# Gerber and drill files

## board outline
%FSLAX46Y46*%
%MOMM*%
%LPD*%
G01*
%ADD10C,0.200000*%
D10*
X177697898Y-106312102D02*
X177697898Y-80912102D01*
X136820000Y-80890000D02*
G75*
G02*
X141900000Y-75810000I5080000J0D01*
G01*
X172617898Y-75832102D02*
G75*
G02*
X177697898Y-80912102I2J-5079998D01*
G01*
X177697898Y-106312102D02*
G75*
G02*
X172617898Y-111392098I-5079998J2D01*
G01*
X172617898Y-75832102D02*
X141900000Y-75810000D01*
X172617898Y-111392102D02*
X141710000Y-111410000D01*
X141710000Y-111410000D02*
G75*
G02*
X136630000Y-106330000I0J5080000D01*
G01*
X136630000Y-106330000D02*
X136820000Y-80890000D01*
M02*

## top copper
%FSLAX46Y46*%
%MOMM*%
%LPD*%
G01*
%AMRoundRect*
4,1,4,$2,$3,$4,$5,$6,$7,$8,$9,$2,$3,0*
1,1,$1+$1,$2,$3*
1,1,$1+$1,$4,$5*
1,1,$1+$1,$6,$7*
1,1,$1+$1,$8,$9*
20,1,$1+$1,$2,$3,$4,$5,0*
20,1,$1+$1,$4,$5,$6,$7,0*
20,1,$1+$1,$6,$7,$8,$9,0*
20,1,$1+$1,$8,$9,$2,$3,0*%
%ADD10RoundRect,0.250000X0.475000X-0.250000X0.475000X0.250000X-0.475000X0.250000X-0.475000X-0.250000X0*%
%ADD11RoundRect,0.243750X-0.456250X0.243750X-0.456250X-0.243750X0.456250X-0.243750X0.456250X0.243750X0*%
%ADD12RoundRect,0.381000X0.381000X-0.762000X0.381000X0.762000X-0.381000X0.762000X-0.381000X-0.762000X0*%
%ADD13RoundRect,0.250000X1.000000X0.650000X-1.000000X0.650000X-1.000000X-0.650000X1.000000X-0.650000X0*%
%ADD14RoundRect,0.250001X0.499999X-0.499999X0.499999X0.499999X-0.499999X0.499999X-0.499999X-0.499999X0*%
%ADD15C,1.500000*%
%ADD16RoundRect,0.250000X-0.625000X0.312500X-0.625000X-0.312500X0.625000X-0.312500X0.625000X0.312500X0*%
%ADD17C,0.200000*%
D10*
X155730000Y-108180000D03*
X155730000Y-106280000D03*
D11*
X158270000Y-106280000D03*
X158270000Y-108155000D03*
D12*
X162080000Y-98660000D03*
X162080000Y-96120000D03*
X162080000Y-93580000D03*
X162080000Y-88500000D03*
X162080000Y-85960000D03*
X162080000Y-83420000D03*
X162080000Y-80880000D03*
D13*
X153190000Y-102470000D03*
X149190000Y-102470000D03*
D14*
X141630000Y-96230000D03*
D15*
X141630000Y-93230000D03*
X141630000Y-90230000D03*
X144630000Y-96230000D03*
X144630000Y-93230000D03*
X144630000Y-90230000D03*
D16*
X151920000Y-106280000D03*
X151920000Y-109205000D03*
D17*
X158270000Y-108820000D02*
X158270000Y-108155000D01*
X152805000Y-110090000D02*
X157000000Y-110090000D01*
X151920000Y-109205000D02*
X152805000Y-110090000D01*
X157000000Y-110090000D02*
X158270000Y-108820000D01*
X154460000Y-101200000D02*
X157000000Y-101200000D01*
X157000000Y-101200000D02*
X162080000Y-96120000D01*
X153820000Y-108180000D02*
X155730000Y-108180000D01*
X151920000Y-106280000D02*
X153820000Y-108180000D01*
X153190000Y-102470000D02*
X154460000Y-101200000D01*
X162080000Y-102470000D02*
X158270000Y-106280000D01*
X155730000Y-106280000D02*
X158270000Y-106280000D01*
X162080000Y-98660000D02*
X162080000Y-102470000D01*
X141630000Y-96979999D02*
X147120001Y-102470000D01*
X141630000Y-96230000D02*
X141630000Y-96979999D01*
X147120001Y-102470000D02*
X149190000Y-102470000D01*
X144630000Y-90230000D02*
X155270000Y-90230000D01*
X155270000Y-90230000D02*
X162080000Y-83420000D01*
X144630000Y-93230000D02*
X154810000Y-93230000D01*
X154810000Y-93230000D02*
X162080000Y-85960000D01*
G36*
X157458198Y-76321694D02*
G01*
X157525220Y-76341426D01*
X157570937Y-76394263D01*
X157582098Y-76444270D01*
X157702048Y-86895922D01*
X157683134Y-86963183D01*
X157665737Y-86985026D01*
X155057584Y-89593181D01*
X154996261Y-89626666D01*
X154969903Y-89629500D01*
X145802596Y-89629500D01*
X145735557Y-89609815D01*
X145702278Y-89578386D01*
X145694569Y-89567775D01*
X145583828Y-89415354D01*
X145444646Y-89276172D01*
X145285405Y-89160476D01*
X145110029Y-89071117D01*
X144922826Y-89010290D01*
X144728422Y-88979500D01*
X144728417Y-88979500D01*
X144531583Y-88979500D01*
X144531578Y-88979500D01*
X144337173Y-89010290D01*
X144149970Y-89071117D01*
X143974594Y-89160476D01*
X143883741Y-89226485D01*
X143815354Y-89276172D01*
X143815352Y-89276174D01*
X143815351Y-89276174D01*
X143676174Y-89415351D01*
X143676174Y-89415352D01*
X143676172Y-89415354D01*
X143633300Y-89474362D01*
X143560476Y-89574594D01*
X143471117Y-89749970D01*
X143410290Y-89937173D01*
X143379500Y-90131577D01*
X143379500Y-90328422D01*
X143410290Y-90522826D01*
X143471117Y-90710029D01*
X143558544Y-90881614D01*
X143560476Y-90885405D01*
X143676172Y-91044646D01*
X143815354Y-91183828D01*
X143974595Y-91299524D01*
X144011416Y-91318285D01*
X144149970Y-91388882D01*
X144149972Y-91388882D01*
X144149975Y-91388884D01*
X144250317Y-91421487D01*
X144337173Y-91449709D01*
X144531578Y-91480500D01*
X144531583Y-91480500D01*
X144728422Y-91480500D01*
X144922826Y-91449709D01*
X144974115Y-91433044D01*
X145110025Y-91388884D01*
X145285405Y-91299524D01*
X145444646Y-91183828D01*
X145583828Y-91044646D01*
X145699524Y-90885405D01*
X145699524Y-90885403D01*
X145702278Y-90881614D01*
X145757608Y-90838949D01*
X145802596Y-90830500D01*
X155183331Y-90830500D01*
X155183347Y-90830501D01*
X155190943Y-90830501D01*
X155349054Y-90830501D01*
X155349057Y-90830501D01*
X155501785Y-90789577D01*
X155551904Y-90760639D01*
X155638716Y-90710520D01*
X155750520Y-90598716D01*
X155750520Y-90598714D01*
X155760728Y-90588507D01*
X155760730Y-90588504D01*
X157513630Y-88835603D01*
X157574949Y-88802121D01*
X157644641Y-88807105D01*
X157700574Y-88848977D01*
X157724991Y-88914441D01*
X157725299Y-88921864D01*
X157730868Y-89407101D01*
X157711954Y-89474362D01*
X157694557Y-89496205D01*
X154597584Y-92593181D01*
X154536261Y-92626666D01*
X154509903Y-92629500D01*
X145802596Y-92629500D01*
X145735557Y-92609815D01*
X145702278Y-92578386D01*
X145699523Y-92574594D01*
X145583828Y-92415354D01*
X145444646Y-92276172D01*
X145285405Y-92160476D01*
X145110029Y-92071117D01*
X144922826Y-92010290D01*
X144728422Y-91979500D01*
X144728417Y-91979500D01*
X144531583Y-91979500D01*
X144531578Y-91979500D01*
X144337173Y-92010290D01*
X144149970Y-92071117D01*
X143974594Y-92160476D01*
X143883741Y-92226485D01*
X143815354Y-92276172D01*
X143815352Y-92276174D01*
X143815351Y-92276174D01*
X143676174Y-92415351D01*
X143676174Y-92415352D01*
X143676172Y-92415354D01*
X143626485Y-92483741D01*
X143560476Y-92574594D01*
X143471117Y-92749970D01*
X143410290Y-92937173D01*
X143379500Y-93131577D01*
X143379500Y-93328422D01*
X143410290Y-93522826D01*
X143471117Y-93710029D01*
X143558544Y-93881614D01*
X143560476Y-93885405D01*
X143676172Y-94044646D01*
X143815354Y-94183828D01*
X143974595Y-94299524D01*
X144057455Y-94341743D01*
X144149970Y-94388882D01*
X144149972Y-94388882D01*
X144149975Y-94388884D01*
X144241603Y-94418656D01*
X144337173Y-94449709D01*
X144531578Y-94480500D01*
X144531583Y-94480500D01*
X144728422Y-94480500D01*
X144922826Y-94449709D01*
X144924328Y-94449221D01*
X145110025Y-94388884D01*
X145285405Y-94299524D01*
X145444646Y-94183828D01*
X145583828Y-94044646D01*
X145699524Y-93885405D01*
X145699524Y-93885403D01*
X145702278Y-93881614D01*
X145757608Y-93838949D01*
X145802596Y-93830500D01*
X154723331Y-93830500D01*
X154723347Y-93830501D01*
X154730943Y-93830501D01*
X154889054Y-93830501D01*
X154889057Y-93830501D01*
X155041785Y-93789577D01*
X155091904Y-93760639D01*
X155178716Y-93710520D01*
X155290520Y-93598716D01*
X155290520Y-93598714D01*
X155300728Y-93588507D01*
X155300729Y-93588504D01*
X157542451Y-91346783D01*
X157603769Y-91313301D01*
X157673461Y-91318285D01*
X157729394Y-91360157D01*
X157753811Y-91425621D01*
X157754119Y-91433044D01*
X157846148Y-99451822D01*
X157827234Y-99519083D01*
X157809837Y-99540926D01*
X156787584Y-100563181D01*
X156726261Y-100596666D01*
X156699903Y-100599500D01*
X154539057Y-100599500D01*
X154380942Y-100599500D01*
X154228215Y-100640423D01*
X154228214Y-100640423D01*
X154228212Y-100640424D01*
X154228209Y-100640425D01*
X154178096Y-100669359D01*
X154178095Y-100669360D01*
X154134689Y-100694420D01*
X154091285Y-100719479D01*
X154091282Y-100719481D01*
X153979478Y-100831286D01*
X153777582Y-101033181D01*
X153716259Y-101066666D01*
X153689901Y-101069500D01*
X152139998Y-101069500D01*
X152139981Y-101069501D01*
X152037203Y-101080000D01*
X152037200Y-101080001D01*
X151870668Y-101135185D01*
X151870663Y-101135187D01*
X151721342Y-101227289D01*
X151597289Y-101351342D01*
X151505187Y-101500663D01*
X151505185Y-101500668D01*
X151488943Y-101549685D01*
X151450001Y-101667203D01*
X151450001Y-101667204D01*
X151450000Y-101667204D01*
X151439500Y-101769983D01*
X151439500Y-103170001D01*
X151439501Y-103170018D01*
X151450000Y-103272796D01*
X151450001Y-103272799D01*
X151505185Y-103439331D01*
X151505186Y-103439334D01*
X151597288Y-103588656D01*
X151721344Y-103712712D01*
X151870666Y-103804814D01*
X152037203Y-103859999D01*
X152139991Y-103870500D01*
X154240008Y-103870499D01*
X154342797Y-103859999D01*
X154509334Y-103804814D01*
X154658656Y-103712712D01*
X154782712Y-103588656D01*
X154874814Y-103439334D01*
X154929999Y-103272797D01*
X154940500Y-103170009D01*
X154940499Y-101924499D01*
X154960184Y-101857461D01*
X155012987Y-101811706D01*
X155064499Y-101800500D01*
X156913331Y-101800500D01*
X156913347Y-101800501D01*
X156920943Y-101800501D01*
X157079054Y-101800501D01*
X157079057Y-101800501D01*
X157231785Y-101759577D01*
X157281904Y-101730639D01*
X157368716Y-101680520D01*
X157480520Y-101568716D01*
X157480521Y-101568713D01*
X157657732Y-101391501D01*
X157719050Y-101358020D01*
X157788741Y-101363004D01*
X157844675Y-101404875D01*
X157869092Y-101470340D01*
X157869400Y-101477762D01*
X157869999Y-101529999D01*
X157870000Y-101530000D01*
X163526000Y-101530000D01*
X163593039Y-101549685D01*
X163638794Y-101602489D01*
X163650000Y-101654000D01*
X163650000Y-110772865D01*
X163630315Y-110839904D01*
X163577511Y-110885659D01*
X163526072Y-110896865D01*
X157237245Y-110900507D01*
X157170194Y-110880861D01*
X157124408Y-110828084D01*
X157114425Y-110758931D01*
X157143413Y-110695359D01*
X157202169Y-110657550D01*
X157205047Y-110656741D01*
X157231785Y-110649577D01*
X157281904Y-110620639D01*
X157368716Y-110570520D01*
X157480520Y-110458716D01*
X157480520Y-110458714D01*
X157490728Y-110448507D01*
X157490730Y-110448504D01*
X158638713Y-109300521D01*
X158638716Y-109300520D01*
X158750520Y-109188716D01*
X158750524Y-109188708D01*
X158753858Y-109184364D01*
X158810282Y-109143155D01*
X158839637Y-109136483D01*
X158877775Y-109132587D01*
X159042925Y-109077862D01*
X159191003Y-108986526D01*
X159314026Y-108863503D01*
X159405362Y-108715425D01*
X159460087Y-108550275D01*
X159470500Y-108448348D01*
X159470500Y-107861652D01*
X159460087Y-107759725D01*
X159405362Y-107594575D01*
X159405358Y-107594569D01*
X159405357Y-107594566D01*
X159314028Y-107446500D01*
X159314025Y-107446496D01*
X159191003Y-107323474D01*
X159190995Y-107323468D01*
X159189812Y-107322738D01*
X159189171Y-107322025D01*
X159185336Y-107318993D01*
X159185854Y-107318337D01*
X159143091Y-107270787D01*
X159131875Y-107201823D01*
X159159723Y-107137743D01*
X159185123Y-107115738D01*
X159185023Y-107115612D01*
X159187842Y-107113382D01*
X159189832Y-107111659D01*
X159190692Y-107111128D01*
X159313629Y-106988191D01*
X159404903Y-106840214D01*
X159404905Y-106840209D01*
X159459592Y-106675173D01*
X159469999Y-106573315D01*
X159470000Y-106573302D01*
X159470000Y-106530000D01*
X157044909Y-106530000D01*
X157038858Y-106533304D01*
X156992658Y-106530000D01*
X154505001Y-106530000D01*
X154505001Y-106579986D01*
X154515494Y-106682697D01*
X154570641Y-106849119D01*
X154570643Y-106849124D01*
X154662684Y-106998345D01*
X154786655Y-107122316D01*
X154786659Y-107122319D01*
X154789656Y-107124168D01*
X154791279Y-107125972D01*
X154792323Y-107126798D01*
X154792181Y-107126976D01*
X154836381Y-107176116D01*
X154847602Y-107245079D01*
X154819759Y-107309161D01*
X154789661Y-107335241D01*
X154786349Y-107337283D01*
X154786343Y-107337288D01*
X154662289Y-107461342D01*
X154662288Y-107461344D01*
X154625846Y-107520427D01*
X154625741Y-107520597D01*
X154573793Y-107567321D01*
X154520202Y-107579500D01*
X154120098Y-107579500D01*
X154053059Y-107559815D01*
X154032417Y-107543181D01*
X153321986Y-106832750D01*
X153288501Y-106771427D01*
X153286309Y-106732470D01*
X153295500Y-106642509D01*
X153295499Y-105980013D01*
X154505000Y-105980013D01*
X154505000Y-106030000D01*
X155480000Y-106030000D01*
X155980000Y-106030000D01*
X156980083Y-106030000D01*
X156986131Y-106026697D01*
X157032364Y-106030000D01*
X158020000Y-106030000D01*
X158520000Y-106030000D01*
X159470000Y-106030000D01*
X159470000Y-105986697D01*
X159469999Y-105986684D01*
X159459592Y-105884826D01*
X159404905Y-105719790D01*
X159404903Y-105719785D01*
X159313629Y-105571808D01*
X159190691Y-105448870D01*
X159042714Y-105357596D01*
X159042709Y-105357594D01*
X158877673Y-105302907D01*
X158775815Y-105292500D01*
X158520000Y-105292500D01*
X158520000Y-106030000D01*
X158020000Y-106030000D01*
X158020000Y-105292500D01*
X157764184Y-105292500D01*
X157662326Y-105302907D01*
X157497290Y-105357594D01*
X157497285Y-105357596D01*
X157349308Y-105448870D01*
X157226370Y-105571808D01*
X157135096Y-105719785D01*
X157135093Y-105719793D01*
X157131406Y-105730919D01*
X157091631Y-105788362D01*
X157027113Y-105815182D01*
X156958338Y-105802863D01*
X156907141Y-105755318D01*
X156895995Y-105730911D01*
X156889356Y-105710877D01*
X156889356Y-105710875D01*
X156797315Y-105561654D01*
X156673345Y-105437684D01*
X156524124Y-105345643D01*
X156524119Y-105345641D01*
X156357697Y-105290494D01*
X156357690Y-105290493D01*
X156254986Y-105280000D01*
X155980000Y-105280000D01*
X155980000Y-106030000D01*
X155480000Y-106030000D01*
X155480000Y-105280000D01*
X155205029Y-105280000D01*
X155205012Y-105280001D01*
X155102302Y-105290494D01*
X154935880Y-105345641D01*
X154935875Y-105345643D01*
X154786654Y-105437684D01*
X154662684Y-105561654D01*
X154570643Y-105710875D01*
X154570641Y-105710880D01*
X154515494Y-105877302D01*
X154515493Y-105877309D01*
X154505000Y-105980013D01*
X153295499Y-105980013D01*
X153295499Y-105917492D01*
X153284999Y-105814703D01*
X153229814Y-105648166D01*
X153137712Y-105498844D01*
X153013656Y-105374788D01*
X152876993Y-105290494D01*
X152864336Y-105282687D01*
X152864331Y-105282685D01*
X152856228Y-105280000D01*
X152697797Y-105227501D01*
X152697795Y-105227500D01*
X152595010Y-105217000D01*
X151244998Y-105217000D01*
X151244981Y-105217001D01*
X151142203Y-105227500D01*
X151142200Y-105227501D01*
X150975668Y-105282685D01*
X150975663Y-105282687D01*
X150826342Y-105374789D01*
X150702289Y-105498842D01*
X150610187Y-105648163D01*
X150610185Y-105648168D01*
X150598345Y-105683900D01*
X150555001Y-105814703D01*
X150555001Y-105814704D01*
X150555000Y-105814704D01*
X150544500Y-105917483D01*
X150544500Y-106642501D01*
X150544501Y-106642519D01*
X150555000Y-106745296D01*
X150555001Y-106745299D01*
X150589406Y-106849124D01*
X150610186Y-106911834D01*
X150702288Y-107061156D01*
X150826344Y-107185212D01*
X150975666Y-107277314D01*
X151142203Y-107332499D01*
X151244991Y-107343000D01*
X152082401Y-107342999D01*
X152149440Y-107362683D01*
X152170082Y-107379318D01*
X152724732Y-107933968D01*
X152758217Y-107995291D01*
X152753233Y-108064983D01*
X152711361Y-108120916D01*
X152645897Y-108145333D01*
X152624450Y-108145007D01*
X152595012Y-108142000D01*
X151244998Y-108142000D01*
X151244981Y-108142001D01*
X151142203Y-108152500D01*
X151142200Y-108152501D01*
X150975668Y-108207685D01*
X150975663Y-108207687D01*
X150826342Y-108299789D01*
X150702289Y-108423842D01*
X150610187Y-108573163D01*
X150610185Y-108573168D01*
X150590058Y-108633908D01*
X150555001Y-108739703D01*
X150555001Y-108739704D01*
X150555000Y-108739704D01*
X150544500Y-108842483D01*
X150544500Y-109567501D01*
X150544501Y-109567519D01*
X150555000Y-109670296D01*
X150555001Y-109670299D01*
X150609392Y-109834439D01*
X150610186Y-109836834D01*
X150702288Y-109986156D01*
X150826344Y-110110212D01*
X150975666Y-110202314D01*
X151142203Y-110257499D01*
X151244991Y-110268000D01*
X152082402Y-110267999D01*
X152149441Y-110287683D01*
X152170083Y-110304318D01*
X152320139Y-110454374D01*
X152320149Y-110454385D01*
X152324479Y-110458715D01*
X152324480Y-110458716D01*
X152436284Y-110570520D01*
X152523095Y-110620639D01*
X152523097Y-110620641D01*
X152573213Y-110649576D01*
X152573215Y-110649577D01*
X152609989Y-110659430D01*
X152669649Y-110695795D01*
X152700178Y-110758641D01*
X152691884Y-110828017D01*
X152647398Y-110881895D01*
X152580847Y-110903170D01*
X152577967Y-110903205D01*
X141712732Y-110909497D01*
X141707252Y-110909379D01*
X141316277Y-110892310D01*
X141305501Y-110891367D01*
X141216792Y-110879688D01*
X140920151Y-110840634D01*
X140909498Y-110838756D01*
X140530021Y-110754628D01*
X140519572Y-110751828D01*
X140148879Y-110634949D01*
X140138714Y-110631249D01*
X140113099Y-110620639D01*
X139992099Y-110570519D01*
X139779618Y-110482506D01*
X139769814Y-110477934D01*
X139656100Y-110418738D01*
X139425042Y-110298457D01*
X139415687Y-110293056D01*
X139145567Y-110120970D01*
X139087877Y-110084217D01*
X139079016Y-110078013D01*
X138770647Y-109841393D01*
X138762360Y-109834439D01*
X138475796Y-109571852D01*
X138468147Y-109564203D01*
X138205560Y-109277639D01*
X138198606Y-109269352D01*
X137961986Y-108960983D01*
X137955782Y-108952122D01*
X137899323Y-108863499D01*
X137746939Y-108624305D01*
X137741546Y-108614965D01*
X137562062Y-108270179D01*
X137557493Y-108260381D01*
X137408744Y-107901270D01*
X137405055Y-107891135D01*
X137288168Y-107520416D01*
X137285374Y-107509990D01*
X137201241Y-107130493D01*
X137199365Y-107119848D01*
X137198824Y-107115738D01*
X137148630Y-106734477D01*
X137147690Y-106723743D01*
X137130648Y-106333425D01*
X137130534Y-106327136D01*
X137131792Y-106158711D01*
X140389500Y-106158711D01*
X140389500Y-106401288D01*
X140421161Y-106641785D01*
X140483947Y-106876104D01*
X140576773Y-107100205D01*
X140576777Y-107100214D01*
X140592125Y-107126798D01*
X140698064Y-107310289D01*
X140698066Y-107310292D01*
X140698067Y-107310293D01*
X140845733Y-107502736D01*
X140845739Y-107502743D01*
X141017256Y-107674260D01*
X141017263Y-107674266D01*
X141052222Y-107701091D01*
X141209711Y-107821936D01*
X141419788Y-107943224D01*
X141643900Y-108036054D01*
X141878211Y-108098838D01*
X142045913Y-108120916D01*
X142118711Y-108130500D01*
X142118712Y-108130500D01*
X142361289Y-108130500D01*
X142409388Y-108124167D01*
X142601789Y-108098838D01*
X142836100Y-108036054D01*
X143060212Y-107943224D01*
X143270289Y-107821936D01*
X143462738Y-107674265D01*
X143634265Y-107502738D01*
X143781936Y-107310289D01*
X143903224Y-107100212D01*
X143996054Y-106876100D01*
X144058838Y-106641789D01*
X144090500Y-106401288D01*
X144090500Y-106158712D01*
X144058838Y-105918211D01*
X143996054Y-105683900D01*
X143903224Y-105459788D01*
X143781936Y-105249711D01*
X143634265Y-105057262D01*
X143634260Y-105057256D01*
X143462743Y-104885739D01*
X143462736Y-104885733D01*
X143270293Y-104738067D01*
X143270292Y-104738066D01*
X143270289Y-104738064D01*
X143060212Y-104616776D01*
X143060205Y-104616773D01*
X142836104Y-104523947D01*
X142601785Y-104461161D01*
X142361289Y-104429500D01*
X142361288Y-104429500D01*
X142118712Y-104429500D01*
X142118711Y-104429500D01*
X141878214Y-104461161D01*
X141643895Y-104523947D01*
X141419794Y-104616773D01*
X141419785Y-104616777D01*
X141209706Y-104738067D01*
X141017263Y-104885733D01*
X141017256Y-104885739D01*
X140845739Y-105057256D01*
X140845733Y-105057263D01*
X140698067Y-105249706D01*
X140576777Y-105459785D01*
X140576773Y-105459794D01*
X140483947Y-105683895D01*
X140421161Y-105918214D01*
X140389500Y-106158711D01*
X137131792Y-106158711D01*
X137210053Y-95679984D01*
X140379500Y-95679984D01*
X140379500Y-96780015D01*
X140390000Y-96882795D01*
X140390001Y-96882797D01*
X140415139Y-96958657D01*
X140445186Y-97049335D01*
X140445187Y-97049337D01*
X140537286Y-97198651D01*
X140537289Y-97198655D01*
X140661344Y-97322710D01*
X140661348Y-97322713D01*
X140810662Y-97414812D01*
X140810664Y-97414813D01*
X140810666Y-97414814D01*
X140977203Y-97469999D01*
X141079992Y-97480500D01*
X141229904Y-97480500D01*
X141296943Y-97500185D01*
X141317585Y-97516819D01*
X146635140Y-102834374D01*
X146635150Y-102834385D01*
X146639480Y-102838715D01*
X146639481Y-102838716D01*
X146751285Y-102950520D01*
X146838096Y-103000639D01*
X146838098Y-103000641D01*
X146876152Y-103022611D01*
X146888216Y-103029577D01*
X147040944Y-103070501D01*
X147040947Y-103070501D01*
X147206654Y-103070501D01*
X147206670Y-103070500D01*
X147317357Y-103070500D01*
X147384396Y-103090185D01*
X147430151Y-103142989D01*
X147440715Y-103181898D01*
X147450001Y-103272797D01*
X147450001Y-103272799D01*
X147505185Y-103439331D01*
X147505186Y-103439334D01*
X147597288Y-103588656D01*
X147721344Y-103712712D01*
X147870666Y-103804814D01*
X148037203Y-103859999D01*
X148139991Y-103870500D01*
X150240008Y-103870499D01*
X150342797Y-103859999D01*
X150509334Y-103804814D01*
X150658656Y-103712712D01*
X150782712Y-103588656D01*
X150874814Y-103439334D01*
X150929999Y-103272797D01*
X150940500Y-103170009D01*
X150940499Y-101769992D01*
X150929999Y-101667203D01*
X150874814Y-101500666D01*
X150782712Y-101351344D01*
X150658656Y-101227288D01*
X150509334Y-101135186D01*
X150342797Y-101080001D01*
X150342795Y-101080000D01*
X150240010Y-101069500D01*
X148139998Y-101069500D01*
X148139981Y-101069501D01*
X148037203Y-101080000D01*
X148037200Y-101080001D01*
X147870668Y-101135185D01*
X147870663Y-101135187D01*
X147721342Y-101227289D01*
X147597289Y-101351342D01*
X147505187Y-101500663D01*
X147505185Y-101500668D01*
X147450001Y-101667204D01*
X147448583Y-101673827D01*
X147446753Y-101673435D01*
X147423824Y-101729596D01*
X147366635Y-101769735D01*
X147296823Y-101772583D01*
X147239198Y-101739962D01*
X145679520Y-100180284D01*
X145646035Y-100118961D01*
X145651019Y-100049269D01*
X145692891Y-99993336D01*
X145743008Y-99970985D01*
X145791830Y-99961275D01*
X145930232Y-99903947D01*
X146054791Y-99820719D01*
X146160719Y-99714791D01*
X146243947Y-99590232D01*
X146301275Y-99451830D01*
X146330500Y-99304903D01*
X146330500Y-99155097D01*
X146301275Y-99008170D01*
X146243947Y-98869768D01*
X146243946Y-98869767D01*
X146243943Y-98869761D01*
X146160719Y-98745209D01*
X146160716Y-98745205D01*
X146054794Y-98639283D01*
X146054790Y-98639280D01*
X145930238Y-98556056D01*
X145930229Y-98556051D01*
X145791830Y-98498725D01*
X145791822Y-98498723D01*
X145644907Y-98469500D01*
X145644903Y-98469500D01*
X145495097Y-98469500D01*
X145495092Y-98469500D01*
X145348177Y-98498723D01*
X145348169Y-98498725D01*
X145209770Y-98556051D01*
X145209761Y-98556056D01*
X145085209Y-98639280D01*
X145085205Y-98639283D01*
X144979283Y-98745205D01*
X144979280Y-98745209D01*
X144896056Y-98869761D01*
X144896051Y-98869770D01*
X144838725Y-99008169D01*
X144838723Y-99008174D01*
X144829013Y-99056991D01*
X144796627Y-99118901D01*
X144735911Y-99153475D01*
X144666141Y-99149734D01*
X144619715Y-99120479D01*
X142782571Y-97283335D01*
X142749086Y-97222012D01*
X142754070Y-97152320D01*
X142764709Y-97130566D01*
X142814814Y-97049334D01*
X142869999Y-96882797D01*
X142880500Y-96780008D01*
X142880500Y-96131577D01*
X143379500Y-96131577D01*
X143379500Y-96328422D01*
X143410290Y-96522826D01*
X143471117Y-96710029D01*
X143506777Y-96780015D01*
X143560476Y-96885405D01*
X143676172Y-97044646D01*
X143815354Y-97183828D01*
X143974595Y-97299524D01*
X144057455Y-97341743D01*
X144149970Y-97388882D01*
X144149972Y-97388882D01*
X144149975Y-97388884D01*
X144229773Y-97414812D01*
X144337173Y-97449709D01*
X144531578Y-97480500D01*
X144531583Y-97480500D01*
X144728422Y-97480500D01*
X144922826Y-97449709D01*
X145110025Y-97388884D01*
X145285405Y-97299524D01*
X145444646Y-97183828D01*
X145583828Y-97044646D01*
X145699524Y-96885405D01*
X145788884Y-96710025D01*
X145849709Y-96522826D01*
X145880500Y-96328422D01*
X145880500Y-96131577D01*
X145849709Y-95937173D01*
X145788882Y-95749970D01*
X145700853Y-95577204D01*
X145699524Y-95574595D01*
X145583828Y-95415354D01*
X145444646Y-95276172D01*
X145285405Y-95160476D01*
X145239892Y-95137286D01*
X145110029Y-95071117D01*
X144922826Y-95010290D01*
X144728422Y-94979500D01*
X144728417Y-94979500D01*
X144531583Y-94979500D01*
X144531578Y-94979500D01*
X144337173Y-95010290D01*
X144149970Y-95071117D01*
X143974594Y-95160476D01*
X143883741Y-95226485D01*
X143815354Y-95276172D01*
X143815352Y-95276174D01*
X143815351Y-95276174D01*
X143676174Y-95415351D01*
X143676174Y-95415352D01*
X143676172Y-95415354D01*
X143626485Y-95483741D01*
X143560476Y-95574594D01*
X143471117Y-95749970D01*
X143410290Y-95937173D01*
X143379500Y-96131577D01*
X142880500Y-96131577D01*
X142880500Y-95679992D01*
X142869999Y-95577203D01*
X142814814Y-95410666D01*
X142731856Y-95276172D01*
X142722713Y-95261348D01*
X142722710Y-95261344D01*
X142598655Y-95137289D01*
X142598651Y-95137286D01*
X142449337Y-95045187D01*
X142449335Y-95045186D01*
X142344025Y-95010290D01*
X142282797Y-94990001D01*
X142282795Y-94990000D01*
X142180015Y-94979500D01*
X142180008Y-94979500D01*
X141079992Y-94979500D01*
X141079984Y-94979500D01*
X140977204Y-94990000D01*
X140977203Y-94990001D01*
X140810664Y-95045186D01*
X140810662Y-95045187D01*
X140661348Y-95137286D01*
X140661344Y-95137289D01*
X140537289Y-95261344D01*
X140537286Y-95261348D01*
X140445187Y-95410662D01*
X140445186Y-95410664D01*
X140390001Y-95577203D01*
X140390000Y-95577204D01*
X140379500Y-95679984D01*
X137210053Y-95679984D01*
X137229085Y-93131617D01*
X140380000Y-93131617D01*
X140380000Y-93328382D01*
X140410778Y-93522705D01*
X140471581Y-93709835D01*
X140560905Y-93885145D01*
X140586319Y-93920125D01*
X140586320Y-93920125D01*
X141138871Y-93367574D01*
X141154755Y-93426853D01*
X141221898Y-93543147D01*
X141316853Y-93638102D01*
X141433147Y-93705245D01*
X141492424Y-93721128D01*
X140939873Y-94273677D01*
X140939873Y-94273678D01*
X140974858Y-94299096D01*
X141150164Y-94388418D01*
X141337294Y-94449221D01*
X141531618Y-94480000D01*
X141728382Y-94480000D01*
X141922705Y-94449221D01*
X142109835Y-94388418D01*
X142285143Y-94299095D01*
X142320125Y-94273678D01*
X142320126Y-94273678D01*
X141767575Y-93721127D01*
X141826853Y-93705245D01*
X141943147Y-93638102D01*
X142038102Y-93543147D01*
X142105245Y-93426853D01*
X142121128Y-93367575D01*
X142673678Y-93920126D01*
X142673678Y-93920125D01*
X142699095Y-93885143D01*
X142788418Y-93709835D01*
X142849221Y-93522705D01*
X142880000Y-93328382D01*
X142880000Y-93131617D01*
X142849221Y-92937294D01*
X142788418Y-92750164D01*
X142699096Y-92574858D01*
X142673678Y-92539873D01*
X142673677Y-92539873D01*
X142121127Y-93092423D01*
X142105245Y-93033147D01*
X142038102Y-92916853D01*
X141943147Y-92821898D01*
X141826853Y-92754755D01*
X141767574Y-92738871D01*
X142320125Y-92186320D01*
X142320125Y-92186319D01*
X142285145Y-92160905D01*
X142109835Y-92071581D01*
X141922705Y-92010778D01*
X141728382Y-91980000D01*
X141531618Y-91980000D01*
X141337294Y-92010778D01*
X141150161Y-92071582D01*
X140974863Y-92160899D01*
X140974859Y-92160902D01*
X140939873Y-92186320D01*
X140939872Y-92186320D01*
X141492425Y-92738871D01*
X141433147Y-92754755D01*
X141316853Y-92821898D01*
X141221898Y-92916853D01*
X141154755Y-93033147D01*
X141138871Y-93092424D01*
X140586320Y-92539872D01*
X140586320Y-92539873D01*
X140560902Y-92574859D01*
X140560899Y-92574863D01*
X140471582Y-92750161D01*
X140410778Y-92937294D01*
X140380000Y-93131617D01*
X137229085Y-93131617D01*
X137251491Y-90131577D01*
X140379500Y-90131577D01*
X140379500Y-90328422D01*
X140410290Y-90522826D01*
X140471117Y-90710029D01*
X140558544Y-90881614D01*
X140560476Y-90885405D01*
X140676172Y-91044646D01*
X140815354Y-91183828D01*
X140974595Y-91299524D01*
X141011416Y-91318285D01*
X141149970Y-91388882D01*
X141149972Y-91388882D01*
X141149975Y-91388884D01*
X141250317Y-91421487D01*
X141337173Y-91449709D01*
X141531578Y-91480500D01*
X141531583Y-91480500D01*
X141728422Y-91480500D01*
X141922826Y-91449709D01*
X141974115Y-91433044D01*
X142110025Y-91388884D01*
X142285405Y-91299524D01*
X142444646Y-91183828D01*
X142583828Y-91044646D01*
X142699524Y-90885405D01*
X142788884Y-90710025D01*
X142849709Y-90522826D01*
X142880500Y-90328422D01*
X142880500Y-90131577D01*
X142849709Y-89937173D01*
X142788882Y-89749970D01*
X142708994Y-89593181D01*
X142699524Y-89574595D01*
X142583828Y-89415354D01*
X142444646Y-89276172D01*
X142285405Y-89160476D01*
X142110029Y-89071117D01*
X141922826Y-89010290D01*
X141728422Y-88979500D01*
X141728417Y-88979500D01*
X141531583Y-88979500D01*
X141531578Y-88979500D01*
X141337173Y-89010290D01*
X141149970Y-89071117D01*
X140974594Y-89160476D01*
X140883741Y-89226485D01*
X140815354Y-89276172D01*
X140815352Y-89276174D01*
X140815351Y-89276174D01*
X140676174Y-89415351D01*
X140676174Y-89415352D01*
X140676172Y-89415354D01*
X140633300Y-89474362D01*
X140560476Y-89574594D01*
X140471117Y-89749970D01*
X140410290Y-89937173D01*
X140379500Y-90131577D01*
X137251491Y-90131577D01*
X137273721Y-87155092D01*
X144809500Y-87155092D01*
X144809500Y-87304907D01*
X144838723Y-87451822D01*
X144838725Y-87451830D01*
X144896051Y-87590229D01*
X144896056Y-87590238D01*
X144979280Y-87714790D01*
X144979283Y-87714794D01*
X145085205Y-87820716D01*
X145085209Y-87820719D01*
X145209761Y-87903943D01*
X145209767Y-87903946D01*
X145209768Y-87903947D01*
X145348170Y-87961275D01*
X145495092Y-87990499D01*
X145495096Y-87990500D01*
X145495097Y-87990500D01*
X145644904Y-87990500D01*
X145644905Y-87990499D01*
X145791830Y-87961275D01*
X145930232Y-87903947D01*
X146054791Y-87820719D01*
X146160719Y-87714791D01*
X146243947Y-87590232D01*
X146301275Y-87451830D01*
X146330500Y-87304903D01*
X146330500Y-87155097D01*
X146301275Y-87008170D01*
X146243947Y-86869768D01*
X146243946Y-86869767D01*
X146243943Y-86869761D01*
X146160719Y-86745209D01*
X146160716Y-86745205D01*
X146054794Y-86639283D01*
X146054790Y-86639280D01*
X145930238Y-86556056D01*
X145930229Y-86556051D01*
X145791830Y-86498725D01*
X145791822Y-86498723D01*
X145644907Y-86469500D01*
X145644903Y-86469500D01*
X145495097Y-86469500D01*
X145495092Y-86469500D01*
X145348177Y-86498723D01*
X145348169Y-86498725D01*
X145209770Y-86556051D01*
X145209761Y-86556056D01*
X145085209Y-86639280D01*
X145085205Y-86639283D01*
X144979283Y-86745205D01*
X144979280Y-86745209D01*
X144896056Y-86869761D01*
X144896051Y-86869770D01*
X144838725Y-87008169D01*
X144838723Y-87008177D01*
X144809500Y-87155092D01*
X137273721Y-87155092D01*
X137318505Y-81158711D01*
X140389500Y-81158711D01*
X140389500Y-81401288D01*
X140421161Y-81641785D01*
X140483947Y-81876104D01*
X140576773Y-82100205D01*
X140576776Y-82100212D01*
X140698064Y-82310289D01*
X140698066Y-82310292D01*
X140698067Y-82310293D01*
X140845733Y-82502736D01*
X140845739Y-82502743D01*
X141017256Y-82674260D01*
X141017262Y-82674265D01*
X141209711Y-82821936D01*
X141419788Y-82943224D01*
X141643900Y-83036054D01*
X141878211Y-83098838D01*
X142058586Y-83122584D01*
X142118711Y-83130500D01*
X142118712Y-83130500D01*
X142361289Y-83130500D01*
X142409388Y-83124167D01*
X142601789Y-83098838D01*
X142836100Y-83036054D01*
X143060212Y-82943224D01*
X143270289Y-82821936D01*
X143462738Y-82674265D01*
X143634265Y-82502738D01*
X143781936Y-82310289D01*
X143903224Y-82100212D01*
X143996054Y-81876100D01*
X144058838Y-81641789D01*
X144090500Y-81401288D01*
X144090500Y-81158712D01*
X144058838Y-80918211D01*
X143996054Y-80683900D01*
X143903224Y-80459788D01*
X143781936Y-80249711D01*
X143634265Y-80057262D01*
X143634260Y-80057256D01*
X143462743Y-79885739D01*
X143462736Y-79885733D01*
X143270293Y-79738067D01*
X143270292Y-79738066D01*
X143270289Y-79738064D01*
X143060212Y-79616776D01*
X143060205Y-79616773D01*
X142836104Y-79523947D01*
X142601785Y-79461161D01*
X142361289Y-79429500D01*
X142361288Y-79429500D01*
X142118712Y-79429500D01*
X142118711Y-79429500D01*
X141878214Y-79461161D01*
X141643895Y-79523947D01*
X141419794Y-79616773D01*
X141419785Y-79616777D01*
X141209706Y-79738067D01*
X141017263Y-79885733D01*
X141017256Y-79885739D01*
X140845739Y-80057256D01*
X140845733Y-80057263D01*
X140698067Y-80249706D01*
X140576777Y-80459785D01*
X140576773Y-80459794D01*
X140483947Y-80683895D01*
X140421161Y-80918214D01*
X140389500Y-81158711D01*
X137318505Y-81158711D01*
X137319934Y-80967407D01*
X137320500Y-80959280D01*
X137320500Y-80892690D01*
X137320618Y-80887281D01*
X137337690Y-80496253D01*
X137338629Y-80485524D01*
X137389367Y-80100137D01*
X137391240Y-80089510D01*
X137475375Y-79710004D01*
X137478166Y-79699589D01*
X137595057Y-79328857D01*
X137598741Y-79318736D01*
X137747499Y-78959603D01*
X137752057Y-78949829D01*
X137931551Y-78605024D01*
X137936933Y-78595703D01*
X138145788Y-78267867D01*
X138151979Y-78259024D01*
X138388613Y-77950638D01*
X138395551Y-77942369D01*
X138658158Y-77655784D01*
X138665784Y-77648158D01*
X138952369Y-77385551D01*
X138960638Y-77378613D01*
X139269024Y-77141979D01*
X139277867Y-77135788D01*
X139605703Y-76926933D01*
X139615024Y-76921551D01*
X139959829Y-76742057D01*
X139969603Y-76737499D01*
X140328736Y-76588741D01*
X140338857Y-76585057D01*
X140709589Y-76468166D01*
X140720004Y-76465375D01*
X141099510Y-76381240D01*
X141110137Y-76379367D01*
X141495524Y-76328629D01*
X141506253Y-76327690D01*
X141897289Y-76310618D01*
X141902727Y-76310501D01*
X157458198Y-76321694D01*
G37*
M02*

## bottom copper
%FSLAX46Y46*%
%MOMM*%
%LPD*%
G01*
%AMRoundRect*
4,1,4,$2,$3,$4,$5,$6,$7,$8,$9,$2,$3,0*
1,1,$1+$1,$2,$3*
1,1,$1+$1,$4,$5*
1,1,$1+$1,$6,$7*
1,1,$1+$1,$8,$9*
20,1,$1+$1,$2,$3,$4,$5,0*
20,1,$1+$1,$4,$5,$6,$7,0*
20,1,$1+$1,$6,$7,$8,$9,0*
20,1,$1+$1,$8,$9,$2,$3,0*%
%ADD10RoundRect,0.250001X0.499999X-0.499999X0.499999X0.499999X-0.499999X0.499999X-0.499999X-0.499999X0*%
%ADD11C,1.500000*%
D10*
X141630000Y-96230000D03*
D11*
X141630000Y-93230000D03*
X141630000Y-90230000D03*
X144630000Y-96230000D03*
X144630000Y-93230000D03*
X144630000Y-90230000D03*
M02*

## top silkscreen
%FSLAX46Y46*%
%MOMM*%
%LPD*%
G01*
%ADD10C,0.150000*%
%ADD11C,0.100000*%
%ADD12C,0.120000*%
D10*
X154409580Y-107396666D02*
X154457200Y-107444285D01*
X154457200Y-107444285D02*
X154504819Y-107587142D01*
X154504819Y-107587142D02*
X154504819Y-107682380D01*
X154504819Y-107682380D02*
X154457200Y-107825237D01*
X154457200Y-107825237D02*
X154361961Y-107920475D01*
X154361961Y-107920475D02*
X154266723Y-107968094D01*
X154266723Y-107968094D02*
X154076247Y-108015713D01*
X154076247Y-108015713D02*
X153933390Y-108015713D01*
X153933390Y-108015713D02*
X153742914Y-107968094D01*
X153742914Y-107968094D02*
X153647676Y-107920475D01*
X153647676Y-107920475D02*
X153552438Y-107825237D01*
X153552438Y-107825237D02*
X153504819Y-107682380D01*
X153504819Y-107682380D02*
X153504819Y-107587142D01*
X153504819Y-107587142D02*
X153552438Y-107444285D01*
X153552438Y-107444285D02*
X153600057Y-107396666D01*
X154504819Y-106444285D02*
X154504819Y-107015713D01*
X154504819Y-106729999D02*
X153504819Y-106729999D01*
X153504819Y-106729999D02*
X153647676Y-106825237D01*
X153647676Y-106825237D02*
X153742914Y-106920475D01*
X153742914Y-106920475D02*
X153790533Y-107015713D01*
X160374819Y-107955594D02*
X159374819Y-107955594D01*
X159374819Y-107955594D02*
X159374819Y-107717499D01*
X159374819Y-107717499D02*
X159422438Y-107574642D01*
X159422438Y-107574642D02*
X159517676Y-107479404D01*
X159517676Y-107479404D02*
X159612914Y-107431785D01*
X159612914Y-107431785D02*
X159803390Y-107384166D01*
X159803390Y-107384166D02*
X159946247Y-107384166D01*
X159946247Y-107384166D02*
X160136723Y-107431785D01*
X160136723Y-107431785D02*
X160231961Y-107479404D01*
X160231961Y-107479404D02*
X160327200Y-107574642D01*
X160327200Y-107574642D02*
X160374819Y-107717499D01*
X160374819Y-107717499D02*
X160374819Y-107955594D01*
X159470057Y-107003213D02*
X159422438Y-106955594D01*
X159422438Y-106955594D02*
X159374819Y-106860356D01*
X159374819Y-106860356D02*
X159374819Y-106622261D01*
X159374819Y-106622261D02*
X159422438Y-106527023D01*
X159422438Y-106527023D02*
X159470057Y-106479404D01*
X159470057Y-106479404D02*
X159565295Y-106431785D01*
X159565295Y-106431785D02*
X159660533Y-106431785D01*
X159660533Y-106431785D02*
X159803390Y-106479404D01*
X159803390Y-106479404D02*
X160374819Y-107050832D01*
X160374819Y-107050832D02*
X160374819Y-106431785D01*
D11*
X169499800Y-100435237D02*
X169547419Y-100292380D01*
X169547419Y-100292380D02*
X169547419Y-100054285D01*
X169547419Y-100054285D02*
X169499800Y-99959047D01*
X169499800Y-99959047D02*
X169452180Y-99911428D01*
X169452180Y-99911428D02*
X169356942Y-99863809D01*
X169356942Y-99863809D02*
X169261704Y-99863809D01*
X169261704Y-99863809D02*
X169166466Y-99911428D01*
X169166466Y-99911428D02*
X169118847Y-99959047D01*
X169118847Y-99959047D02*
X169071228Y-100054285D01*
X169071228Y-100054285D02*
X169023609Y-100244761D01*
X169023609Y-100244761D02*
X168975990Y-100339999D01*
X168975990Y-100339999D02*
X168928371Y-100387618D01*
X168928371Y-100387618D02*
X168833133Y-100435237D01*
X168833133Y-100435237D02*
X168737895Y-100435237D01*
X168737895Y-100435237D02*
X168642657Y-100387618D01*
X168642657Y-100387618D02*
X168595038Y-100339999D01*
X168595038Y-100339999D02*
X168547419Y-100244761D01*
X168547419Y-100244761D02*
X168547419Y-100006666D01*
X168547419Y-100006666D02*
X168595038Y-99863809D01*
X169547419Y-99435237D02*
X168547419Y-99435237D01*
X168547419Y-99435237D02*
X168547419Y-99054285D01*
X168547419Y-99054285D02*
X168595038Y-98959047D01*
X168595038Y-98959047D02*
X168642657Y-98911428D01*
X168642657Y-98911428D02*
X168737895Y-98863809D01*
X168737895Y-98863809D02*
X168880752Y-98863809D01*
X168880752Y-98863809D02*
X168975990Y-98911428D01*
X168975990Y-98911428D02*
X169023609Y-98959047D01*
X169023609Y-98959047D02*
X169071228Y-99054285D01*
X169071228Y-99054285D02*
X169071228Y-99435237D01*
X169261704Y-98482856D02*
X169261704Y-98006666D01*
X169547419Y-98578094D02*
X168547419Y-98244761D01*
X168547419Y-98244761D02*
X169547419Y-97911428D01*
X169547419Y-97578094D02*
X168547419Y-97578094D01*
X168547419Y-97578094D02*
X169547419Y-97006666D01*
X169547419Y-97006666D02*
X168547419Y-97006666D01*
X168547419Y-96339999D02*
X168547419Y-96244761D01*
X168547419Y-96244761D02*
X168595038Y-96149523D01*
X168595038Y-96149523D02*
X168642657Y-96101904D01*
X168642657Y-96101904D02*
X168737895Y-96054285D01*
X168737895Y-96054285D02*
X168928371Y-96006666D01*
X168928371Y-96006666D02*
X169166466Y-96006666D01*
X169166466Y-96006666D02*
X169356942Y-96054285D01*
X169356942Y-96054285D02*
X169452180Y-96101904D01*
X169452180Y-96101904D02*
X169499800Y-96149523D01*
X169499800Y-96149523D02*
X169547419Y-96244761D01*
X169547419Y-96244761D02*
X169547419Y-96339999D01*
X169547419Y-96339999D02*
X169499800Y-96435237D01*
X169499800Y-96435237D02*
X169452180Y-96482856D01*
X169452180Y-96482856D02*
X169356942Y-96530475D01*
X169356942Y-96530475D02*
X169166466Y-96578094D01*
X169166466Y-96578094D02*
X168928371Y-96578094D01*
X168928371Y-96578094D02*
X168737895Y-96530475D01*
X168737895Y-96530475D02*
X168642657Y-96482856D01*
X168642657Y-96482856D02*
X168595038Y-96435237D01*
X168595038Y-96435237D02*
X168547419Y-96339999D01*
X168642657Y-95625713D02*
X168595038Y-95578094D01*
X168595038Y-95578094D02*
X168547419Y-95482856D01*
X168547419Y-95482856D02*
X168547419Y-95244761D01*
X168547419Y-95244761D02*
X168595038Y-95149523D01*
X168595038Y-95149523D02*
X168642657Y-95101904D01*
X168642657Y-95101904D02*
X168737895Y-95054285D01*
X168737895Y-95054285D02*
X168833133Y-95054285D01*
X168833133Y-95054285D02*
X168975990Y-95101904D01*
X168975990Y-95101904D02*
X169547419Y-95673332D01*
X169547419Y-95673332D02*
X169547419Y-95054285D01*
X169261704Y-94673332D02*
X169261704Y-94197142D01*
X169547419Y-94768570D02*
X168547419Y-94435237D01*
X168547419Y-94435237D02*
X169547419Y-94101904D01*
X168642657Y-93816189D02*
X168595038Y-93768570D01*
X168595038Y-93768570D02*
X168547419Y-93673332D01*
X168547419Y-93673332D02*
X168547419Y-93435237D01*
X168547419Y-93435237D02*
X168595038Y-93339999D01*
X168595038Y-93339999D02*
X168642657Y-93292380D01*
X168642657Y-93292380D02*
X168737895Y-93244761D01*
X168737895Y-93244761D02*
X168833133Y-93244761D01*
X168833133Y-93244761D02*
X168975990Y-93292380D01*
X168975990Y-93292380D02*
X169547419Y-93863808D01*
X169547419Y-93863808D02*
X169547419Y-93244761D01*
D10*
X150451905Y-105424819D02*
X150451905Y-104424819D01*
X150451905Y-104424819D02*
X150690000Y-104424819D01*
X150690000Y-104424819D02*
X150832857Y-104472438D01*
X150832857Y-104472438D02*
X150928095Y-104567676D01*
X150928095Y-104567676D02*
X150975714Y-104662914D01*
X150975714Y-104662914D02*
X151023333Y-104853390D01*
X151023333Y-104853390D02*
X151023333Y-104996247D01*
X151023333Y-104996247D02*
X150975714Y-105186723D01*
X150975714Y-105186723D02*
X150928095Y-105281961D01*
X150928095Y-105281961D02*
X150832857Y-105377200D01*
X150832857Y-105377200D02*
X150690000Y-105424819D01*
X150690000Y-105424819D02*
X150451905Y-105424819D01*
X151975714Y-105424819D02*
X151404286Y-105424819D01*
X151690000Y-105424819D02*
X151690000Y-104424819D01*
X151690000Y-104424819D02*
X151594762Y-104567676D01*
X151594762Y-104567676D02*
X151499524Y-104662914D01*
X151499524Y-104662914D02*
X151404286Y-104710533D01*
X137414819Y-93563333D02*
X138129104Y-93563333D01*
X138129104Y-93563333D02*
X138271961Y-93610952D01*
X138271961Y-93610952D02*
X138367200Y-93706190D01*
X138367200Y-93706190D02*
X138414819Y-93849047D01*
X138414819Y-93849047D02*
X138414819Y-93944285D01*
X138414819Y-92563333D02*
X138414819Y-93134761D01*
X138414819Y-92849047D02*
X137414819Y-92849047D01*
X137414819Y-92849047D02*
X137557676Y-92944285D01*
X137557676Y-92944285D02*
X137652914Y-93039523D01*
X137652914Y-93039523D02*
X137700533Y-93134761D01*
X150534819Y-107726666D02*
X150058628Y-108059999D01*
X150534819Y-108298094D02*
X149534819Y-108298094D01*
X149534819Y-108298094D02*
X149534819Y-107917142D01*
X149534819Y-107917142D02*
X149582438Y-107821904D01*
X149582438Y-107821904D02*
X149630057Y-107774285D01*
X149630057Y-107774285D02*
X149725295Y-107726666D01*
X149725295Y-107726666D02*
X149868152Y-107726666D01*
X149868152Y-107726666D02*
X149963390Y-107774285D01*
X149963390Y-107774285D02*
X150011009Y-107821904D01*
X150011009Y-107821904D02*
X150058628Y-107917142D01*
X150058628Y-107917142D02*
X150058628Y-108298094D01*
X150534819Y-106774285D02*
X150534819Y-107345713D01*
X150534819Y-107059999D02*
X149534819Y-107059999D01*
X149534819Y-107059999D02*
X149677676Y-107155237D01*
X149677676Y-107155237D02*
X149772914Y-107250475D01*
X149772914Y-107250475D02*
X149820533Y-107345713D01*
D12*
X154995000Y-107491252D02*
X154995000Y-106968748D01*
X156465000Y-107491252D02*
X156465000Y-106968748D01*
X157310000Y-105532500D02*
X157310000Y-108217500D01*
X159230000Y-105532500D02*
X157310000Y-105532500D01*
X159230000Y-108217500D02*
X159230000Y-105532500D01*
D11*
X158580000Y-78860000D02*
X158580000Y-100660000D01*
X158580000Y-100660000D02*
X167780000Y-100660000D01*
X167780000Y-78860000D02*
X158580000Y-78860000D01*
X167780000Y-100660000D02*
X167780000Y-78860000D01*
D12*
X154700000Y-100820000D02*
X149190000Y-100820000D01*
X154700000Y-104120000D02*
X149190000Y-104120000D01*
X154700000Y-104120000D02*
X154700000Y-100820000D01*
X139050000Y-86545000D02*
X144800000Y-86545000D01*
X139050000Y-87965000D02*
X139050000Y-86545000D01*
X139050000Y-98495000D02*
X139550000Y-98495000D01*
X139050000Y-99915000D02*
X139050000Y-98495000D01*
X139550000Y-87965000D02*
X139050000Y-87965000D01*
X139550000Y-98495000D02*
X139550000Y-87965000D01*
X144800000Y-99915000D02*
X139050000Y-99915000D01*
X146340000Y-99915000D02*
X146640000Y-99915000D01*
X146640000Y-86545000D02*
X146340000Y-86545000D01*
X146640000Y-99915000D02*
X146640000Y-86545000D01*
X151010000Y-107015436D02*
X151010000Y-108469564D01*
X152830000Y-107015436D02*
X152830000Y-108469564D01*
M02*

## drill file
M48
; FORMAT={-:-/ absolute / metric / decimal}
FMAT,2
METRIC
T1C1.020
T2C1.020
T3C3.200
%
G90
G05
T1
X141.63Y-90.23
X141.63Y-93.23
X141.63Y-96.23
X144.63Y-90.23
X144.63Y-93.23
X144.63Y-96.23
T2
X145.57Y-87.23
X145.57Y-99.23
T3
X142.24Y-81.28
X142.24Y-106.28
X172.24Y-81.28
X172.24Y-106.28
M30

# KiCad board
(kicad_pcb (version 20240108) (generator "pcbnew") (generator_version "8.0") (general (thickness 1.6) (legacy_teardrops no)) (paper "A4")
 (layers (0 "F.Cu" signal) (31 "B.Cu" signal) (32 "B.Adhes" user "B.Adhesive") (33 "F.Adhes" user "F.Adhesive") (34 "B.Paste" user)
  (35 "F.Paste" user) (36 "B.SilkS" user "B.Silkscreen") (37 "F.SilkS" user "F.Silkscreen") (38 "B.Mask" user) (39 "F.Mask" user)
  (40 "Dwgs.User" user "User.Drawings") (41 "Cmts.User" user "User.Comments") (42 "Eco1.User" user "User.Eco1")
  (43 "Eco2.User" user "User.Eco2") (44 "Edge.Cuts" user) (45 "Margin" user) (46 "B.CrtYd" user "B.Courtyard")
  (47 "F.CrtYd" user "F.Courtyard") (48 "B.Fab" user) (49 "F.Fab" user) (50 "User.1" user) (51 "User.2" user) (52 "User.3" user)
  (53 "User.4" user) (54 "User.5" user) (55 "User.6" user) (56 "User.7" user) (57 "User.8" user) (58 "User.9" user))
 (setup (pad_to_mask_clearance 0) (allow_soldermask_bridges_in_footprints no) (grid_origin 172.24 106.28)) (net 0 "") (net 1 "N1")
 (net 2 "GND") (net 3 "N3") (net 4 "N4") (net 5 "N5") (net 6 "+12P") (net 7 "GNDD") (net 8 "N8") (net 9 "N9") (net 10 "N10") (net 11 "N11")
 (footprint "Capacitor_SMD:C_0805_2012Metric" (layer "F.Cu") (at 155.73 107.23 90)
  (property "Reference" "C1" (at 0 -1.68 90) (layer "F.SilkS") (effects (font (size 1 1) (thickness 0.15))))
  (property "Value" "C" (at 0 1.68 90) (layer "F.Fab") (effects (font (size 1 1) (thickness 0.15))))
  (fp_line (start -0.261252 -0.735) (end 0.261252 -0.735) (stroke (width 0.12) (type solid)) (layer "F.SilkS"))
  (fp_line (start -0.261252 0.735) (end 0.261252 0.735) (stroke (width 0.12) (type solid)) (layer "F.SilkS"))
  (pad "1" smd roundrect (at -0.95 0 90) (size 1 1.45) (layers "F.Cu" "F.Paste" "F.Mask") (roundrect_rratio 0.25) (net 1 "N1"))
  (pad "2" smd roundrect (at 0.95 0 90) (size 1 1.45) (layers "F.Cu" "F.Paste" "F.Mask") (roundrect_rratio 0.25) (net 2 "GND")))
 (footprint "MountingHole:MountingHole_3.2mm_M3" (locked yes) (layer "F.Cu") (at 142.24 81.28)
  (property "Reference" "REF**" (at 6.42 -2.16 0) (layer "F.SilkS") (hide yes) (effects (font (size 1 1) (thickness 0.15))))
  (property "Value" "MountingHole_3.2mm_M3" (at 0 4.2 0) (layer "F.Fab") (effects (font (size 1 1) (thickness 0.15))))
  (pad "" np_thru_hole circle (at 0 0) (size 3.2 3.2) (drill 3.2) (layers "F&B.Cu" "*.Mask")))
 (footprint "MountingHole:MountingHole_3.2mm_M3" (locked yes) (layer "F.Cu") (at 172.24 106.28)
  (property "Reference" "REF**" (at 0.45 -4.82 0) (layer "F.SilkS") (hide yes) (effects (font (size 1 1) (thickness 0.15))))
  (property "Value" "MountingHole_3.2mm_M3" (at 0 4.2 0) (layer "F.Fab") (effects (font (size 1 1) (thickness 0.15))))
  (pad "" np_thru_hole circle (at 0 0) (size 3.2 3.2) (drill 3.2) (layers "F&B.Cu" "*.Mask")))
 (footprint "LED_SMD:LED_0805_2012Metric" (layer "F.Cu") (at 158.27 107.2175 -90)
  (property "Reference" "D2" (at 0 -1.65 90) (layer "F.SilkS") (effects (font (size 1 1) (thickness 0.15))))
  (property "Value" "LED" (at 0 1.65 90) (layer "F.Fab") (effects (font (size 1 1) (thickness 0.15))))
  (fp_line (start -1.685 0.96) (end 1 0.96) (stroke (width 0.12) (type solid)) (layer "F.SilkS"))
  (fp_line (start -1.685 -0.96) (end -1.685 0.96) (stroke (width 0.12) (type solid)) (layer "F.SilkS"))
  (fp_line (start 1 -0.96) (end -1.685 -0.96) (stroke (width 0.12) (type solid)) (layer "F.SilkS"))
  (pad "1" smd roundrect (at -0.9375 0 270) (size 0.975 1.4) (layers "F.Cu" "F.Paste" "F.Mask") (roundrect_rratio 0.25) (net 2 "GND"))
  (pad "2" smd roundrect (at 0.9375 0 270) (size 0.975 1.4) (layers "F.Cu" "F.Paste" "F.Mask") (roundrect_rratio 0.25) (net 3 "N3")))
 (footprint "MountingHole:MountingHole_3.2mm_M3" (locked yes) (layer "F.Cu") (at 142.24 106.28)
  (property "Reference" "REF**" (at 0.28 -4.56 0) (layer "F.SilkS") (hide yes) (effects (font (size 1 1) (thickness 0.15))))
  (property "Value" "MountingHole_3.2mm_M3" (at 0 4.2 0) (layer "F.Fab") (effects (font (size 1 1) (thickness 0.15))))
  (pad "" np_thru_hole circle (at 0 0) (size 3.2 3.2) (drill 3.2) (layers "F&B.Cu" "*.Mask")))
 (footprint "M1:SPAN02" (layer "F.Cu") (at 162.08 98.66 90)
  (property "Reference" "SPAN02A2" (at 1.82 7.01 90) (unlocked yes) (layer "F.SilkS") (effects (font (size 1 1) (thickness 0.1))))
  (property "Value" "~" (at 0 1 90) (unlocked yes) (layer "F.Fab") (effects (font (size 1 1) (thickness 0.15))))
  (fp_line (start 19.8 -3.5) (end -2 -3.5) (stroke (width 0.1) (type default)) (layer "F.SilkS"))
  (fp_line (start -2 -3.5) (end -2 5.7) (stroke (width 0.1) (type default)) (layer "F.SilkS"))
  (fp_line (start 19.8 5.7) (end 19.8 -3.5) (stroke (width 0.1) (type default)) (layer "F.SilkS"))
  (fp_line (start -2 5.7) (end 19.8 5.7) (stroke (width 0.1) (type default)) (layer "F.SilkS"))
  (pad "1" smd roundrect (at 0 0 90) (size 2.286 1.524) (layers "F.Cu" "F.Paste" "F.Mask") (roundrect_rratio 0.25) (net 2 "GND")
   (thermal_bridge_angle 45))
  (pad "2" smd roundrect (at 2.54 0 90) (size 2.286 1.524) (layers "F.Cu" "F.Paste" "F.Mask") (roundrect_rratio 0.25) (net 1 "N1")
   (thermal_bridge_angle 45))
  (pad "3" smd roundrect (at 5.08 0 90) (size 2.286 1.524) (layers "F.Cu" "F.Paste" "F.Mask") (roundrect_rratio 0.25) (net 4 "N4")
   (thermal_bridge_angle 45))
  (pad "5" smd roundrect (at 10.16 0 90) (size 2.286 1.524) (layers "F.Cu" "F.Paste" "F.Mask") (roundrect_rratio 0.25) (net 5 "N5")
   (thermal_bridge_angle 45))
  (pad "6" smd roundrect (at 12.7 0 90) (size 2.286 1.524) (layers "F.Cu" "F.Paste" "F.Mask") (roundrect_rratio 0.25) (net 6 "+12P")
   (thermal_bridge_angle 45))
  (pad "7" smd roundrect (at 15.24 0 90) (size 2.286 1.524) (layers "F.Cu" "F.Paste" "F.Mask") (roundrect_rratio 0.25) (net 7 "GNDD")
   (thermal_bridge_angle 45))
  (pad "8" smd roundrect (at 17.78 0 90) (size 2.286 1.524) (layers "F.Cu" "F.Paste" "F.Mask") (roundrect_rratio 0.25) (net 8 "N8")
   (thermal_bridge_angle 45)))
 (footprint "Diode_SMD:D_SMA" (layer "F.Cu") (at 151.19 102.47 180)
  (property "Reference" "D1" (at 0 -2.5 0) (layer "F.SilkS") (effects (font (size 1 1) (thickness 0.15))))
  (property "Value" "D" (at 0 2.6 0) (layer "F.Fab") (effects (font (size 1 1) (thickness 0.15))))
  (fp_line (start -3.51 1.65) (end 2 1.65) (stroke (width 0.12) (type solid)) (layer "F.SilkS"))
  (fp_line (start -3.51 -1.65) (end 2 -1.65) (stroke (width 0.12) (type solid)) (layer "F.SilkS"))
  (fp_line (start -3.51 -1.65) (end -3.51 1.65) (stroke (width 0.12) (type solid)) (layer "F.SilkS"))
  (pad "1" smd roundrect (at -2 0 180) (size 2.5 1.8) (layers "F.Cu" "F.Paste" "F.Mask") (roundrect_rratio 0.1388888889) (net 1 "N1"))
  (pad "2" smd roundrect (at 2 0 180) (size 2.5 1.8) (layers "F.Cu" "F.Paste" "F.Mask") (roundrect_rratio 0.1388888889) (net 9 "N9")))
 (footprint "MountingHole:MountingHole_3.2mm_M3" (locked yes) (layer "F.Cu") (at 172.24 81.28)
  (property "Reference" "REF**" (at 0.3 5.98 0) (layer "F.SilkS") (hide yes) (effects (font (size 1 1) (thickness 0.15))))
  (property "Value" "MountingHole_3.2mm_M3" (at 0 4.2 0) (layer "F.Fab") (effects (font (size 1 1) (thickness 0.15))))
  (pad "" np_thru_hole circle (at 0 0) (size 3.2 3.2) (drill 3.2) (layers "F&B.Cu" "*.Mask")))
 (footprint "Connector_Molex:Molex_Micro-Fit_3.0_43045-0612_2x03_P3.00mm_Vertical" (layer "F.Cu") (at 141.63 96.23 90)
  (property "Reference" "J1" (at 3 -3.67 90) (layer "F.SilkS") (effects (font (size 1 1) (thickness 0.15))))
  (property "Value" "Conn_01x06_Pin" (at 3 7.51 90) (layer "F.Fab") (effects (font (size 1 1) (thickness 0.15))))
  (fp_line (start 9.685 -2.58) (end 9.685 3.17) (stroke (width 0.12) (type solid)) (layer "F.SilkS"))
  (fp_line (start 8.265 -2.58) (end 9.685 -2.58) (stroke (width 0.12) (type solid)) (layer "F.SilkS"))
  (fp_line (start -2.265 -2.58) (end -2.265 -2.08) (stroke (width 0.12) (type solid)) (layer "F.SilkS"))
  (fp_line (start -3.685 -2.58) (end -2.265 -2.58) (stroke (width 0.12) (type solid)) (layer "F.SilkS"))
  (fp_line (start 8.265 -2.08) (end 8.265 -2.58) (stroke (width 0.12) (type solid)) (layer "F.SilkS"))
  (fp_line (start -2.265 -2.08) (end 8.265 -2.08) (stroke (width 0.12) (type solid)) (layer "F.SilkS"))
  (fp_line (start -3.685 3.17) (end -3.685 -2.58) (stroke (width 0.12) (type solid)) (layer "F.SilkS"))
  (fp_line (start -3.685 4.71) (end -3.685 5.01) (stroke (width 0.12) (type solid)) (layer "F.SilkS"))
  (fp_line (start 9.685 5.01) (end 9.685 4.71) (stroke (width 0.12) (type solid)) (layer "F.SilkS"))
  (fp_line (start -3.685 5.01) (end 9.685 5.01) (stroke (width 0.12) (type solid)) (layer "F.SilkS"))
  (pad "" np_thru_hole circle (at -3 3.94 90) (size 1.02 1.02) (drill 1.02) (layers "*.Cu" "*.Mask"))
  (pad "" np_thru_hole circle (at 9 3.94 90) (size 1.02 1.02) (drill 1.02) (layers "*.Cu" "*.Mask"))
  (pad "1" thru_hole roundrect (at 0 0 90) (size 1.5 1.5) (drill 1.02) (layers "*.Cu" "*.Mask") (remove_unused_layers no)
   (roundrect_rratio 0.166667) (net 9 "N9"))
  (pad "2" thru_hole circle (at 3 0 90) (size 1.5 1.5) (drill 1.02) (layers "*.Cu" "*.Mask") (remove_unused_layers no) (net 2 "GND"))
  (pad "3" thru_hole circle (at 6 0 90) (size 1.5 1.5) (drill 1.02) (layers "*.Cu" "*.Mask") (remove_unused_layers no) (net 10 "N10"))
  (pad "4" thru_hole circle (at 0 3 90) (size 1.5 1.5) (drill 1.02) (layers "*.Cu" "*.Mask") (remove_unused_layers no) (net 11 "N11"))
  (pad "5" thru_hole circle (at 3 3 90) (size 1.5 1.5) (drill 1.02) (layers "*.Cu" "*.Mask") (remove_unused_layers no) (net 6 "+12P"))
  (pad "6" thru_hole circle (at 6 3 90) (size 1.5 1.5) (drill 1.02) (layers "*.Cu" "*.Mask") (remove_unused_layers no) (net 7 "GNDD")))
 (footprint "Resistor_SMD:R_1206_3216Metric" (layer "F.Cu") (at 151.92 107.7425 -90)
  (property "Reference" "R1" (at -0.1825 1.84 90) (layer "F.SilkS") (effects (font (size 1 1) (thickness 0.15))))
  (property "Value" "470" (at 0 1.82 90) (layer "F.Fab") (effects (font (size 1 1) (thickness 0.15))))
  (fp_line (start -0.727064 0.91) (end 0.727064 0.91) (stroke (width 0.12) (type solid)) (layer "F.SilkS"))
  (fp_line (start -0.727064 -0.91) (end 0.727064 -0.91) (stroke (width 0.12) (type solid)) (layer "F.SilkS"))
  (pad "1" smd roundrect (at -1.4625 0 270) (size 1.125 1.75) (layers "F.Cu" "F.Paste" "F.Mask") (roundrect_rratio 0.222222) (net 1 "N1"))
  (pad "2" smd roundrect (at 1.4625 0 270) (size 1.125 1.75) (layers "F.Cu" "F.Paste" "F.Mask") (roundrect_rratio 0.222222) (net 3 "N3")))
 (gr_line (start 177.697898 106.312102) (end 177.697898 80.912102) (stroke (width 0.2) (type default)) (layer "Edge.Cuts"))
 (gr_arc (start 136.82 80.89) (mid 138.307898 77.297898) (end 141.9 75.81) (stroke (width 0.2) (type default)) (layer "Edge.Cuts"))
 (gr_arc (start 172.617898 75.832102) (mid 176.21 77.32) (end 177.697898 80.912102) (stroke (width 0.2) (type default)) (layer "Edge.Cuts"))
 (gr_arc (start 177.697898 106.312102) (mid 176.21 109.904204) (end 172.617898 111.392102) (stroke (width 0.2) (type default))
  (layer "Edge.Cuts"))
 (gr_line (start 172.617898 75.832102) (end 141.9 75.81) (stroke (width 0.2) (type default)) (layer "Edge.Cuts"))
 (gr_line (start 172.617898 111.392102) (end 141.71 111.41) (stroke (width 0.2) (type default)) (layer "Edge.Cuts"))
 (gr_arc (start 141.71 111.41) (mid 138.117898 109.922102) (end 136.63 106.33) (stroke (width 0.2) (type default)) (layer "Edge.Cuts"))
 (gr_line (start 136.63 106.33) (end 136.82 80.89) (stroke (width 0.2) (type default)) (layer "Edge.Cuts"))
 (segment (start 158.27 108.82) (end 158.27 108.155) (width 0.2) (layer "F.Cu") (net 3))
 (segment (start 152.805 110.09) (end 157 110.09) (width 0.2) (layer "F.Cu") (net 3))
 (segment (start 151.92 109.205) (end 152.805 110.09) (width 0.2) (layer "F.Cu") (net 3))
 (segment (start 157 110.09) (end 158.27 108.82) (width 0.2) (layer "F.Cu") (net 3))
 (segment (start 154.46 101.2) (end 157 101.2) (width 0.2) (layer "F.Cu") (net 1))
 (segment (start 157 101.2) (end 162.08 96.12) (width 0.2) (layer "F.Cu") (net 1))
 (segment (start 153.82 108.18) (end 155.73 108.18) (width 0.2) (layer "F.Cu") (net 1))
 (segment (start 151.92 106.28) (end 153.82 108.18) (width 0.2) (layer "F.Cu") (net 1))
 (segment (start 153.19 102.47) (end 154.46 101.2) (width 0.2) (layer "F.Cu") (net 1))
 (segment (start 162.08 102.47) (end 158.27 106.28) (width 0.2) (layer "F.Cu") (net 2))
 (segment (start 155.73 106.28) (end 158.27 106.28) (width 0.2) (layer "F.Cu") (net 2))
 (segment (start 162.08 98.66) (end 162.08 102.47) (width 0.2) (layer "F.Cu") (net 2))
 (segment (start 141.63 96.979999) (end 147.120001 102.47) (width 0.2) (layer "F.Cu") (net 9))
 (segment (start 141.63 96.23) (end 141.63 96.979999) (width 0.2) (layer "F.Cu") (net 9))
 (segment (start 147.120001 102.47) (end 149.19 102.47) (width 0.2) (layer "F.Cu") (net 9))
 (segment (start 144.63 90.23) (end 155.27 90.23) (width 0.2) (layer "F.Cu") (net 7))
 (segment (start 155.27 90.23) (end 162.08 83.42) (width 0.2) (layer "F.Cu") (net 7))
 (segment (start 144.63 93.23) (end 154.81 93.23) (width 0.2) (layer "F.Cu") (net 6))
 (segment (start 154.81 93.23) (end 162.08 85.96) (width 0.2) (layer "F.Cu") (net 6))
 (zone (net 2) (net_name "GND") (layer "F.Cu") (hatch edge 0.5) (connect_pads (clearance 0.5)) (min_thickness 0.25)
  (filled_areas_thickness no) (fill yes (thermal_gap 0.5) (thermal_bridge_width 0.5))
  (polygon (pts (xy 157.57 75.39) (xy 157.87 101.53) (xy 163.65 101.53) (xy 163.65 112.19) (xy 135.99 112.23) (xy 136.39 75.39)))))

